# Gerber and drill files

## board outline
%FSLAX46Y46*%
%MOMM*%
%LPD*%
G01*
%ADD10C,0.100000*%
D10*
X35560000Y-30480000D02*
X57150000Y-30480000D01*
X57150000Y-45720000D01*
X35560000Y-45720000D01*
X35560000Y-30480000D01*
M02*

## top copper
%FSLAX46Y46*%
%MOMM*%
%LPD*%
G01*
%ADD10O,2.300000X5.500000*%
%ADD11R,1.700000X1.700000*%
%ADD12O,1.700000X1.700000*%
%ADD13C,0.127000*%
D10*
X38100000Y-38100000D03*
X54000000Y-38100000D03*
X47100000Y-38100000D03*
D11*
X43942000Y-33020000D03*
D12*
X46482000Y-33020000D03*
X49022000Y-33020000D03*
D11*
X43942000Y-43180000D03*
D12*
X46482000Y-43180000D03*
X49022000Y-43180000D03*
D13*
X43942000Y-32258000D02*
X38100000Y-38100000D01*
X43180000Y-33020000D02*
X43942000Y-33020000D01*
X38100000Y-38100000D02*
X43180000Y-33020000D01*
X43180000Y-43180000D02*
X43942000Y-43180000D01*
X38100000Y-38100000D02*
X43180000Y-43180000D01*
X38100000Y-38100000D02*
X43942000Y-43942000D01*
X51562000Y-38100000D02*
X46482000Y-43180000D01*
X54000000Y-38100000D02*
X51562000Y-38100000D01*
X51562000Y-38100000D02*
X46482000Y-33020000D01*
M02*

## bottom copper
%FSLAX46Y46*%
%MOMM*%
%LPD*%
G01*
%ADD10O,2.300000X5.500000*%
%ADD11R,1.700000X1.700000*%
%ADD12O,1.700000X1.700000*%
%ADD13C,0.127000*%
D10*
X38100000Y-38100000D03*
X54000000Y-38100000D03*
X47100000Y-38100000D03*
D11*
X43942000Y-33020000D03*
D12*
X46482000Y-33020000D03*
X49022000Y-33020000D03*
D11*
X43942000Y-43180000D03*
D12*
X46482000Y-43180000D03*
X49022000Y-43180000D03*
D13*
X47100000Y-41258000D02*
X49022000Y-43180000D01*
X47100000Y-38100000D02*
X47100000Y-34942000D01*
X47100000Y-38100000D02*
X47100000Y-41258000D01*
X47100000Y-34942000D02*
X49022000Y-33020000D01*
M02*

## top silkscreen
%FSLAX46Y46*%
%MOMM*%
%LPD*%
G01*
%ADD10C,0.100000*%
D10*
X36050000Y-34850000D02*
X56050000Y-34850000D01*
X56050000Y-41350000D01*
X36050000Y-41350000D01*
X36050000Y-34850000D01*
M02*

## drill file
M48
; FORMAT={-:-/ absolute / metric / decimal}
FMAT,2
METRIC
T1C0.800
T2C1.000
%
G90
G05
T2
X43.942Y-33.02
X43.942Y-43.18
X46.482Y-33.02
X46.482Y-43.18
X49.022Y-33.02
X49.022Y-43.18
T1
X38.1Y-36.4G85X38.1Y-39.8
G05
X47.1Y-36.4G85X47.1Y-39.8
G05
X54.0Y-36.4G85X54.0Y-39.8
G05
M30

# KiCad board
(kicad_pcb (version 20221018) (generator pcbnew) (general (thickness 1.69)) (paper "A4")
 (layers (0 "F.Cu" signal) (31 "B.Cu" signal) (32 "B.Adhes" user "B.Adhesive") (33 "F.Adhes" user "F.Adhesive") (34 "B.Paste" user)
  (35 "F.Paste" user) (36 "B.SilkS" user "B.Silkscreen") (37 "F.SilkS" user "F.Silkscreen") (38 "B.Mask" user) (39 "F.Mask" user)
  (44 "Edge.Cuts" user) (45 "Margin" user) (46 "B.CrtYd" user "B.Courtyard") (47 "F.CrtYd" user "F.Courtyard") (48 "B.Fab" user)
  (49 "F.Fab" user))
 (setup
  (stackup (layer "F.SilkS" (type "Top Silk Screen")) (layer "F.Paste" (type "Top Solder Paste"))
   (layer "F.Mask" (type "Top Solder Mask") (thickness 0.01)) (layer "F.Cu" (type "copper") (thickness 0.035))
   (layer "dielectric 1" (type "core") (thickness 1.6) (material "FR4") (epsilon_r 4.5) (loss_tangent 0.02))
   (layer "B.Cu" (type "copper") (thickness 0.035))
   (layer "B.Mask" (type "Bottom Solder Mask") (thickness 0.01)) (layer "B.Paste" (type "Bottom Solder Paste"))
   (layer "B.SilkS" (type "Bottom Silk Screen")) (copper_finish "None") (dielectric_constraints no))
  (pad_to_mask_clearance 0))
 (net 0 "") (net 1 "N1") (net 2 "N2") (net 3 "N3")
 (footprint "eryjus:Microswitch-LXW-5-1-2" (layer "F.Cu") (at 46.05 38.1)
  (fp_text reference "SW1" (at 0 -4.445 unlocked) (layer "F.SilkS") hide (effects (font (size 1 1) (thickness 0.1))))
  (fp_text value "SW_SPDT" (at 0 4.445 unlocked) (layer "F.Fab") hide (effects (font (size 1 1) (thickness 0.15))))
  (fp_rect (start -10 -3.25) (end 10 3.25) (stroke (width 0.1) (type default)) (fill none) (layer "F.SilkS"))
  (pad "1" thru_hole oval (at -7.95 0) (size 2.3 5.5) (drill oval 0.8 4.2) (layers "*.Cu" "*.Mask") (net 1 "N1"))
  (pad "2" thru_hole oval (at 7.95 0) (size 2.3 5.5) (drill oval 0.8 4.2) (layers "*.Cu" "*.Mask") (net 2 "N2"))
  (pad "3" thru_hole oval (at 1.05 0) (size 2.3 5.5) (drill oval 0.8 4.2) (layers "*.Cu" "*.Mask") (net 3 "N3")))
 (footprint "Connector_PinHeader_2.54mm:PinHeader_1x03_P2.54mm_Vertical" (layer "B.Cu") (at 43.942 33.02 -90)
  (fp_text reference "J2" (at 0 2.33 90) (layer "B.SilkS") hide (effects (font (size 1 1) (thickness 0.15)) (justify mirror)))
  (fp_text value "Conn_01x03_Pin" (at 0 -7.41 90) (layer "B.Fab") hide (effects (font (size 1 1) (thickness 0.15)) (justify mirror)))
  (pad "1" thru_hole rect (at 0 0 270) (size 1.7 1.7) (drill 1) (layers "*.Cu" "*.Mask") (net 1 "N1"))
  (pad "2" thru_hole oval (at 0 -2.54 270) (size 1.7 1.7) (drill 1) (layers "*.Cu" "*.Mask") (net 2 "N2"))
  (pad "3" thru_hole oval (at 0 -5.08 270) (size 1.7 1.7) (drill 1) (layers "*.Cu" "*.Mask") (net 3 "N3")))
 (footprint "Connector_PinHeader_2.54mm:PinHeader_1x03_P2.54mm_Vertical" (layer "B.Cu") (at 43.942 43.18 -90)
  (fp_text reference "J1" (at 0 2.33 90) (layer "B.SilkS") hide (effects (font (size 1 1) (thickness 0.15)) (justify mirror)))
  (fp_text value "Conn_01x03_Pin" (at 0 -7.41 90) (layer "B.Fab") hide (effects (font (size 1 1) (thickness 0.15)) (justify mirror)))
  (pad "1" thru_hole rect (at 0 0 270) (size 1.7 1.7) (drill 1) (layers "*.Cu" "*.Mask") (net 1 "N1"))
  (pad "2" thru_hole oval (at 0 -2.54 270) (size 1.7 1.7) (drill 1) (layers "*.Cu" "*.Mask") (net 2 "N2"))
  (pad "3" thru_hole oval (at 0 -5.08 270) (size 1.7 1.7) (drill 1) (layers "*.Cu" "*.Mask") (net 3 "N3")))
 (gr_rect (start 35.56 30.48) (end 57.15 45.72) (stroke (width 0.1) (type default)) (fill none) (layer "Edge.Cuts"))
 (segment (start 43.942 32.258) (end 38.1 38.1) (width 0.127) (layer "F.Cu") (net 1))
 (segment (start 43.18 33.02) (end 43.942 33.02) (width 0.127) (layer "F.Cu") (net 1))
 (segment (start 38.1 38.1) (end 43.18 33.02) (width 0.127) (layer "F.Cu") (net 1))
 (segment (start 43.18 43.18) (end 43.942 43.18) (width 0.127) (layer "F.Cu") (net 1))
 (segment (start 38.1 38.1) (end 43.18 43.18) (width 0.127) (layer "F.Cu") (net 1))
 (segment (start 38.1 38.1) (end 43.942 43.942) (width 0.127) (layer "F.Cu") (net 1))
 (segment (start 51.562 38.1) (end 46.482 43.18) (width 0.127) (layer "F.Cu") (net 2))
 (segment (start 54 38.1) (end 51.562 38.1) (width 0.127) (layer "F.Cu") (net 2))
 (segment (start 51.562 38.1) (end 46.482 33.02) (width 0.127) (layer "F.Cu") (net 2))
 (segment (start 47.1 41.258) (end 49.022 43.18) (width 0.127) (layer "B.Cu") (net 3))
 (segment (start 47.1 38.1) (end 47.1 34.942) (width 0.127) (layer "B.Cu") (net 3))
 (segment (start 47.1 38.1) (end 47.1 41.258) (width 0.127) (layer "B.Cu") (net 3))
 (segment (start 47.1 34.942) (end 49.022 33.02) (width 0.127) (layer "B.Cu") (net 3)))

